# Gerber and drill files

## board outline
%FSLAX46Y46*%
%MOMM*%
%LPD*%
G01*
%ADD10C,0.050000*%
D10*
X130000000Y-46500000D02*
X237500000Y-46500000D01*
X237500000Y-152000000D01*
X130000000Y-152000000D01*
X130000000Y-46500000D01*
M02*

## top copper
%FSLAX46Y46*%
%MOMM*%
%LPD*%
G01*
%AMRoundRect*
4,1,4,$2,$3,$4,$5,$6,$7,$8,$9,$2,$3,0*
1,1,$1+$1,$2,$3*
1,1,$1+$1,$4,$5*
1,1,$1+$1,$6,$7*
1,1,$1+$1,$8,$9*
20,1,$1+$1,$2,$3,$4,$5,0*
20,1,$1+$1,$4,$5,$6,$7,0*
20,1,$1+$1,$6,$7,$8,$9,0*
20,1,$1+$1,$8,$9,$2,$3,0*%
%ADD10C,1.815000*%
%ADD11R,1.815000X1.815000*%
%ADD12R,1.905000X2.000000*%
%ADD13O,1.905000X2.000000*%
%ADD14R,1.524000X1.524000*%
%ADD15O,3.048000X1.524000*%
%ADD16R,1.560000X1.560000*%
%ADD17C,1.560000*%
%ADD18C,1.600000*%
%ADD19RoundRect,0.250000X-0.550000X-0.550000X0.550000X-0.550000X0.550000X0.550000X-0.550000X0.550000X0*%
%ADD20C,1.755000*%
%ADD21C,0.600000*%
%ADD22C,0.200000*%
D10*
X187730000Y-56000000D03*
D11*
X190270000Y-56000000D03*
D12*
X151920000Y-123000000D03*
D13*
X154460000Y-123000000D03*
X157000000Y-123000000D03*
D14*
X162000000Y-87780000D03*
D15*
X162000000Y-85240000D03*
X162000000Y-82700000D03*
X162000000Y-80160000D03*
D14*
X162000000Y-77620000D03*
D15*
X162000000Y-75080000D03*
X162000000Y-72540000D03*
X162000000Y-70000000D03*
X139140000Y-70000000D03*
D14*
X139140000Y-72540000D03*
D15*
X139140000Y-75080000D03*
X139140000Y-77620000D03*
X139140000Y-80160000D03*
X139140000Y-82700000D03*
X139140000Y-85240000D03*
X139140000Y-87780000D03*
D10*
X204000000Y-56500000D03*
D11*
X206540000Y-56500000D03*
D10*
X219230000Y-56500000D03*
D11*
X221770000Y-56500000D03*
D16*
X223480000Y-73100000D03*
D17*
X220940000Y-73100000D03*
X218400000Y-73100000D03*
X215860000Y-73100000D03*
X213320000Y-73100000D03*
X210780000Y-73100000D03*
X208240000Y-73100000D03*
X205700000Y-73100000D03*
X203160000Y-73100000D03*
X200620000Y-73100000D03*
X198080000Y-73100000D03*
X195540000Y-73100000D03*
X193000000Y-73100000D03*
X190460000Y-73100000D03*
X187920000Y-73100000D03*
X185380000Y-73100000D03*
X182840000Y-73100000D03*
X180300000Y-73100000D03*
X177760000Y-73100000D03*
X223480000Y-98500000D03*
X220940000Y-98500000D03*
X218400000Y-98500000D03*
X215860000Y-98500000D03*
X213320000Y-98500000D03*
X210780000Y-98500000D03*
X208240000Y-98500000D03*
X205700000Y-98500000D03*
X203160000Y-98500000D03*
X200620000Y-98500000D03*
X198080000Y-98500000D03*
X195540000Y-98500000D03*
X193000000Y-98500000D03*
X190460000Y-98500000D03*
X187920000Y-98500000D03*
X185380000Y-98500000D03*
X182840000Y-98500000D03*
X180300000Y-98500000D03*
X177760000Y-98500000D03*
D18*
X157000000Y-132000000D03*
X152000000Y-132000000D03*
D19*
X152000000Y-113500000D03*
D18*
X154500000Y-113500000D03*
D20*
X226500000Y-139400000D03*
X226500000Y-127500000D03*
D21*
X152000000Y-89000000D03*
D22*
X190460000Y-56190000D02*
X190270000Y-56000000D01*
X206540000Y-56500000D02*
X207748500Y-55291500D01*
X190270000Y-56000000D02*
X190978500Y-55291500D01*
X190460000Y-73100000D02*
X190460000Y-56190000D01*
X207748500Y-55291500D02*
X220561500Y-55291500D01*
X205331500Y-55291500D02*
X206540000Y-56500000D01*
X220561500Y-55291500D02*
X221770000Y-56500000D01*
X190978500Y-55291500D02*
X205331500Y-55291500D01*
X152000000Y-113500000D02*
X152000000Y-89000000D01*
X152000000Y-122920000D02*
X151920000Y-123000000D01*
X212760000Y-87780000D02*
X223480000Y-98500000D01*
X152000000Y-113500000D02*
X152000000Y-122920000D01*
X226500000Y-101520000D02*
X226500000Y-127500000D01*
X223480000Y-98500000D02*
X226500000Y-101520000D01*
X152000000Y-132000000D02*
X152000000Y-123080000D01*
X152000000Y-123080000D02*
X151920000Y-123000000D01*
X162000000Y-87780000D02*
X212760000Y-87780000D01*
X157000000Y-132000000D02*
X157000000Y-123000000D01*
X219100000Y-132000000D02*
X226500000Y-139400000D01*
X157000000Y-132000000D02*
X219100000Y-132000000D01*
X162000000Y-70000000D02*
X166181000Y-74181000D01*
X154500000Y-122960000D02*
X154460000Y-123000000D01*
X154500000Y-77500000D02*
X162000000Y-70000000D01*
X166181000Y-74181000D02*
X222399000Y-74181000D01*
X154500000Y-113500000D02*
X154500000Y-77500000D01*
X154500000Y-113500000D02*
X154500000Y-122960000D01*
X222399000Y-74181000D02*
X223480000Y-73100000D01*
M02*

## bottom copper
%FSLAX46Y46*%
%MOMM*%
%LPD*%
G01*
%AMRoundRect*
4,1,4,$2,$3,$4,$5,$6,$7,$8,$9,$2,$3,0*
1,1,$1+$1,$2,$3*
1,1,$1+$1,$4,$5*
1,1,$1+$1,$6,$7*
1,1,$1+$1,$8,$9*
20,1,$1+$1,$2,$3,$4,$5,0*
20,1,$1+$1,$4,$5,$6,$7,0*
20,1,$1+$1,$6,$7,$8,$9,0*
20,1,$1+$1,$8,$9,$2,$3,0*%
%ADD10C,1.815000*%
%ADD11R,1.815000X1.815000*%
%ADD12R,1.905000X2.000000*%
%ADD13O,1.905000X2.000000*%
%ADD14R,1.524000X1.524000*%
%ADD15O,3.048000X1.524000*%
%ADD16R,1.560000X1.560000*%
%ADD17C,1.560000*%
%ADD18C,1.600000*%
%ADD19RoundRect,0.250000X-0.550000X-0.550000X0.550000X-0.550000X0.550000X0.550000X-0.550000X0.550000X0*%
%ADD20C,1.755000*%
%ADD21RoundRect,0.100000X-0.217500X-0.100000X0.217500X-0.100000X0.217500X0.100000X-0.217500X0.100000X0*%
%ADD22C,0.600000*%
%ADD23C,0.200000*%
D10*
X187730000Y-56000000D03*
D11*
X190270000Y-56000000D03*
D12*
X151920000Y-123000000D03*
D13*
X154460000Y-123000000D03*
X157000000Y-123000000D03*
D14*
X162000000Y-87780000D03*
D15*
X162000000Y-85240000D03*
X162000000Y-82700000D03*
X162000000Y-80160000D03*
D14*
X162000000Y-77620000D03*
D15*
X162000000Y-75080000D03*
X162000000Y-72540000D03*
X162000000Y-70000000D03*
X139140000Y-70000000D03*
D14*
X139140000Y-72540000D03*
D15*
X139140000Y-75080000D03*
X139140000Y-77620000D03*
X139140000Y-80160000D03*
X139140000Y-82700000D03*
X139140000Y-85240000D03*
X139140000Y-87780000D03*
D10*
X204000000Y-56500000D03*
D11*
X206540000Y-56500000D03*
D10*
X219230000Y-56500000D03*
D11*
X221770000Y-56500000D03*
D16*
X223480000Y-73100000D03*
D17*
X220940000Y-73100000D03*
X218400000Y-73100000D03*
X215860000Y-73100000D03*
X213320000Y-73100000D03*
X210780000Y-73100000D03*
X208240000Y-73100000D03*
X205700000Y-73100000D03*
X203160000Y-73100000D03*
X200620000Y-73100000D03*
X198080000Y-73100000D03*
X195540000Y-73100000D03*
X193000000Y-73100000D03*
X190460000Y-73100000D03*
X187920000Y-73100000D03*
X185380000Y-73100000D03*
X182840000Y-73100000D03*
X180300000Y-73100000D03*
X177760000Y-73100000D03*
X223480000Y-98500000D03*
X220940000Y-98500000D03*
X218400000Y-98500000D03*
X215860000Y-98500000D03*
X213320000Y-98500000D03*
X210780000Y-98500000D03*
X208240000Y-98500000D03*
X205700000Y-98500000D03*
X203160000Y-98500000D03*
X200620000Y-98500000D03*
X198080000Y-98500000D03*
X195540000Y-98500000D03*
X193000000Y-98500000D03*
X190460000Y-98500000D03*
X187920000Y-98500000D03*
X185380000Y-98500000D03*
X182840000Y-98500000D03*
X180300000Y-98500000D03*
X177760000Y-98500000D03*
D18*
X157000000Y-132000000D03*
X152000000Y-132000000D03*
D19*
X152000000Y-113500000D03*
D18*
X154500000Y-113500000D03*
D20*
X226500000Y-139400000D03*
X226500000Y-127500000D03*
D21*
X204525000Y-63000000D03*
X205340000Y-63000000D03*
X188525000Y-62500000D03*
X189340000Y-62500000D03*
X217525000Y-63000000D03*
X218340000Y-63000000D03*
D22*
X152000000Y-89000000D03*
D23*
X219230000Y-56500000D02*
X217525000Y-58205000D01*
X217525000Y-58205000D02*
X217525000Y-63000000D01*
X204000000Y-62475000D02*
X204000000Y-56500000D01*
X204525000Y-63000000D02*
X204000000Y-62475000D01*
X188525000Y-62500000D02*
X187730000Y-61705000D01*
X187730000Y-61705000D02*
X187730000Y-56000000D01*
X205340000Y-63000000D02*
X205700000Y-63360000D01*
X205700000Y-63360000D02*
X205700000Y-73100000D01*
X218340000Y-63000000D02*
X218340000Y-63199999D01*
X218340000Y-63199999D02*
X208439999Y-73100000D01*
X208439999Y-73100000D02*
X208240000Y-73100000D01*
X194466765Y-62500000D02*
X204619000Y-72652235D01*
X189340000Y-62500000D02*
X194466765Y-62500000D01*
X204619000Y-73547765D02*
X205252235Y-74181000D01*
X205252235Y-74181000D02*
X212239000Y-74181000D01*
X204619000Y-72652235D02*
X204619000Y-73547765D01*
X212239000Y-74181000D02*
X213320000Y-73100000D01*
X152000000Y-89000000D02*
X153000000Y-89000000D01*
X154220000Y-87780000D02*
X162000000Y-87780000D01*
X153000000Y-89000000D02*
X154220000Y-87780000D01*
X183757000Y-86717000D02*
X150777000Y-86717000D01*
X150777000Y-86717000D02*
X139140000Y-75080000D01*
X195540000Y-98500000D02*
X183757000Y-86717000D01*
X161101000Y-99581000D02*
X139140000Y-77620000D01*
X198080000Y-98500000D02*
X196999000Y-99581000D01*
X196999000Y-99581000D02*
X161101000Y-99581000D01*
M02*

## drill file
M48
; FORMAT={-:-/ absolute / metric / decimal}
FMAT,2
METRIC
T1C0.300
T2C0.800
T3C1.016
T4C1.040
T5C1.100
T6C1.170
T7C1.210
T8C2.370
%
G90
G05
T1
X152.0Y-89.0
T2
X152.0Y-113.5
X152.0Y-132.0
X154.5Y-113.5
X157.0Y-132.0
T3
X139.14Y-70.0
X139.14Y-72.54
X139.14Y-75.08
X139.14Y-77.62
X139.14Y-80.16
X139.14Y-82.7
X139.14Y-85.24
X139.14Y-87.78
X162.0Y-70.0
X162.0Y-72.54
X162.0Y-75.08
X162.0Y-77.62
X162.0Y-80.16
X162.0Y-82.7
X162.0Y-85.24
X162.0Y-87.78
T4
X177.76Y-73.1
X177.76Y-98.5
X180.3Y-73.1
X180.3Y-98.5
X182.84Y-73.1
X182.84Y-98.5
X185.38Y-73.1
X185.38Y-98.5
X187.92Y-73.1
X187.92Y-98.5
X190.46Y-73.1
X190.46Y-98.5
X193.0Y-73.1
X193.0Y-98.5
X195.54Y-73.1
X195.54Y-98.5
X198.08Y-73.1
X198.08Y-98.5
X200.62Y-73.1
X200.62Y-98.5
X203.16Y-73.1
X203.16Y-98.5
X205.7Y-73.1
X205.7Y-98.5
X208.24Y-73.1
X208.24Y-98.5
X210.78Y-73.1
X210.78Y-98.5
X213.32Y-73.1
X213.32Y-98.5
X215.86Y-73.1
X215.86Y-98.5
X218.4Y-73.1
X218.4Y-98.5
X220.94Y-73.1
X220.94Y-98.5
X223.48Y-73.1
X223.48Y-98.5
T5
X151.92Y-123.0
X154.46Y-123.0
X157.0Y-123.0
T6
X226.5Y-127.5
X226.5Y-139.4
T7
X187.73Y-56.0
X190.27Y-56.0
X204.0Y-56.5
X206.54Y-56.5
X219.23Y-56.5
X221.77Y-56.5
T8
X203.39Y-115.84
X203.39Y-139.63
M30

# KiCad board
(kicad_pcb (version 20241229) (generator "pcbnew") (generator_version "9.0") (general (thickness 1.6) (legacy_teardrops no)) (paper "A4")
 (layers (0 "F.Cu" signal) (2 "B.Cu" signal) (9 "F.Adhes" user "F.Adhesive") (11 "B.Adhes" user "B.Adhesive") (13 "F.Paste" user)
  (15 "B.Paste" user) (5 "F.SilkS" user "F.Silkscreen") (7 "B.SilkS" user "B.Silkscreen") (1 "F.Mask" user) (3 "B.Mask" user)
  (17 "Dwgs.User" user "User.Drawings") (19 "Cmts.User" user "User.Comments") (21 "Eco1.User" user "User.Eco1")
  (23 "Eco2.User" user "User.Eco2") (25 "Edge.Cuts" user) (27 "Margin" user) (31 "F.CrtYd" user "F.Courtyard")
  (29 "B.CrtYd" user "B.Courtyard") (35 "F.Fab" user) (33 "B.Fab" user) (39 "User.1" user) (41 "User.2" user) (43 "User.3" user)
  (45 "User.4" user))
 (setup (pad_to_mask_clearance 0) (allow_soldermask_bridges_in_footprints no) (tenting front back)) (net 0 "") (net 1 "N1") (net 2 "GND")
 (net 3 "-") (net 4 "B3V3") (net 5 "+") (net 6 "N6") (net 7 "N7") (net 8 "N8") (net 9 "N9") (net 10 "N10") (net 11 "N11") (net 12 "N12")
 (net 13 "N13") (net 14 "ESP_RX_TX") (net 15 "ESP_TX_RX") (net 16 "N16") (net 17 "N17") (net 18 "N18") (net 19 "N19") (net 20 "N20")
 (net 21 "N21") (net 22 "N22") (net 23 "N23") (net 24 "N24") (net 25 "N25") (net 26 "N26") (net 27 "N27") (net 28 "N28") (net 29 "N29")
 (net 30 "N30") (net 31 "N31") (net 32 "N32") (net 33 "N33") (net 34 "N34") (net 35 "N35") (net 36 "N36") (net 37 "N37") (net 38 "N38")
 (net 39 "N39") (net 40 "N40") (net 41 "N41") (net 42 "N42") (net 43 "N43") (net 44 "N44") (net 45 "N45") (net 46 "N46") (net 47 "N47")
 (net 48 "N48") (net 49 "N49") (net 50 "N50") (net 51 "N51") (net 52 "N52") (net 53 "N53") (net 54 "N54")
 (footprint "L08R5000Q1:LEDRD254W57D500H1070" (layer "F.Cu") (at 189 56 180)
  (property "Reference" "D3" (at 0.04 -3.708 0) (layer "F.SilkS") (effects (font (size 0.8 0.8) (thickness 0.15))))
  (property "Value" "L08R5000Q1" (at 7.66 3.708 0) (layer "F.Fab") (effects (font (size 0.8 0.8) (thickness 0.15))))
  (pad "A" thru_hole circle (at 1.27 0 180) (size 1.815 1.815) (drill 1.21) (layers "*.Cu" "*.Mask") (remove_unused_layers no) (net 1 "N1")
   (solder_mask_margin 0.102))
  (pad "C" thru_hole rect (at -1.27 0 180) (size 1.815 1.815) (drill 1.21) (layers "*.Cu" "*.Mask") (remove_unused_layers no) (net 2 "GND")
   (solder_mask_margin 0.102)))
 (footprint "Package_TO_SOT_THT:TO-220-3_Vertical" (layer "F.Cu") (at 151.92 123)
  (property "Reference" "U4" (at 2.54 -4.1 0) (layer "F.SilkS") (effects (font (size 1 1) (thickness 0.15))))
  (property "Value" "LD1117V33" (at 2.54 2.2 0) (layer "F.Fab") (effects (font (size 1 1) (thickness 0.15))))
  (pad "1" thru_hole rect (at 0 0) (size 1.905 2) (drill 1.1) (layers "*.Cu" "*.Mask") (remove_unused_layers no) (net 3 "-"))
  (pad "2" thru_hole oval (at 2.54 0) (size 1.905 2) (drill 1.1) (layers "*.Cu" "*.Mask") (remove_unused_layers no) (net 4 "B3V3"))
  (pad "3" thru_hole oval (at 5.08 0) (size 1.905 2) (drill 1.1) (layers "*.Cu" "*.Mask") (remove_unused_layers no) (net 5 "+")))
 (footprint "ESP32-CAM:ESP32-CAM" (layer "F.Cu") (at 150.57 80.16 180)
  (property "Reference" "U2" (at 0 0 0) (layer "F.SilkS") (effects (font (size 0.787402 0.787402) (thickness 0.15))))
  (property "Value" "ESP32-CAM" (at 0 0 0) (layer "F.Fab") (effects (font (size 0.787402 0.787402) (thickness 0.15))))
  (pad "P$1" thru_hole rect (at -11.43 -7.62 180) (size 1.524 1.524) (drill 1.016) (layers "*.Cu" "*.Mask") (remove_unused_layers no)
   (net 3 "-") (solder_mask_margin 0.102))
  (pad "P$2" thru_hole oval (at -11.43 -5.08 180) (size 3.048 1.524) (drill 1.016) (layers "*.Cu" "*.Mask") (remove_unused_layers no)
   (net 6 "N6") (solder_mask_margin 0.102))
  (pad "P$3" thru_hole oval (at -11.43 -2.54 180) (size 3.048 1.524) (drill 1.016) (layers "*.Cu" "*.Mask") (remove_unused_layers no)
   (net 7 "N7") (solder_mask_margin 0.102))
  (pad "P$4" thru_hole oval (at -11.43 0 180) (size 3.048 1.524) (drill 1.016) (layers "*.Cu" "*.Mask") (remove_unused_layers no)
   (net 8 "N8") (solder_mask_margin 0.102))
  (pad "P$5" thru_hole rect (at -11.43 2.54 180) (size 1.524 1.524) (drill 1.016) (layers "*.Cu" "*.Mask") (remove_unused_layers no)
   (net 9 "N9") (solder_mask_margin 0.102))
  (pad "P$6" thru_hole oval (at -11.43 5.08 180) (size 3.048 1.524) (drill 1.016) (layers "*.Cu" "*.Mask") (remove_unused_layers no)
   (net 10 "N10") (solder_mask_margin 0.102))
  (pad "P$7" thru_hole oval (at -11.43 7.62 180) (size 3.048 1.524) (drill 1.016) (layers "*.Cu" "*.Mask") (remove_unused_layers no)
   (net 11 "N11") (solder_mask_margin 0.102))
  (pad "P$8" thru_hole oval (at -11.43 10.16 180) (size 3.048 1.524) (drill 1.016) (layers "*.Cu" "*.Mask") (remove_unused_layers no)
   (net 4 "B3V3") (solder_mask_margin 0.102))
  (pad "P$9" thru_hole oval (at 11.43 10.16 180) (size 3.048 1.524) (drill 1.016) (layers "*.Cu" "*.Mask") (remove_unused_layers no)
   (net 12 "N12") (solder_mask_margin 0.102))
  (pad "P$10" thru_hole rect (at 11.43 7.62 180) (size 1.524 1.524) (drill 1.016) (layers "*.Cu" "*.Mask") (remove_unused_layers no)
   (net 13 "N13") (solder_mask_margin 0.102))
  (pad "P$11" thru_hole oval (at 11.43 5.08 180) (size 3.048 1.524) (drill 1.016) (layers "*.Cu" "*.Mask") (remove_unused_layers no)
   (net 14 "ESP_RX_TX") (solder_mask_margin 0.102))
  (pad "P$12" thru_hole oval (at 11.43 2.54 180) (size 3.048 1.524) (drill 1.016) (layers "*.Cu" "*.Mask") (remove_unused_layers no)
   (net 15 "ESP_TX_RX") (solder_mask_margin 0.102))
  (pad "P$13" thru_hole oval (at 11.43 0 180) (size 3.048 1.524) (drill 1.016) (layers "*.Cu" "*.Mask") (remove_unused_layers no)
   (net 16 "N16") (solder_mask_margin 0.102))
  (pad "P$14" thru_hole oval (at 11.43 -2.54 180) (size 3.048 1.524) (drill 1.016) (layers "*.Cu" "*.Mask") (remove_unused_layers no)
   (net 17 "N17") (solder_mask_margin 0.102))
  (pad "P$15" thru_hole oval (at 11.43 -5.08 180) (size 3.048 1.524) (drill 1.016) (layers "*.Cu" "*.Mask") (remove_unused_layers no)
   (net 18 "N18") (solder_mask_margin 0.102))
  (pad "P$16" thru_hole oval (at 11.43 -7.62 180) (size 3.048 1.524) (drill 1.016) (layers "*.Cu" "*.Mask") (remove_unused_layers no)
   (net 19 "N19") (solder_mask_margin 0.102)))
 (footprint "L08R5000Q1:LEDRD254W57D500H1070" (layer "F.Cu") (at 205.27 56.5 180)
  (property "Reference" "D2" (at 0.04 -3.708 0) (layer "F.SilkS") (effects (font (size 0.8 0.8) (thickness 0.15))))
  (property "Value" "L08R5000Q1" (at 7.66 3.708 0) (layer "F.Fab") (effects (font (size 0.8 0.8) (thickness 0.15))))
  (pad "A" thru_hole circle (at 1.27 0 180) (size 1.815 1.815) (drill 1.21) (layers "*.Cu" "*.Mask") (remove_unused_layers no)
   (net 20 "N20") (solder_mask_margin 0.102))
  (pad "C" thru_hole rect (at -1.27 0 180) (size 1.815 1.815) (drill 1.21) (layers "*.Cu" "*.Mask") (remove_unused_layers no) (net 2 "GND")
   (solder_mask_margin 0.102)))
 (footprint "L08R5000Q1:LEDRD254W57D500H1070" (layer "F.Cu") (at 220.5 56.5 180)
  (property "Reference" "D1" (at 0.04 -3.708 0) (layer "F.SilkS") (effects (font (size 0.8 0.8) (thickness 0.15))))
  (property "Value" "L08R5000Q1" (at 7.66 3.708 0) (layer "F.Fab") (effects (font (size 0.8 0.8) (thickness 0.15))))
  (pad "A" thru_hole circle (at 1.27 0 180) (size 1.815 1.815) (drill 1.21) (layers "*.Cu" "*.Mask") (remove_unused_layers no)
   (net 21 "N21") (solder_mask_margin 0.102))
  (pad "C" thru_hole rect (at -1.27 0 180) (size 1.815 1.815) (drill 1.21) (layers "*.Cu" "*.Mask") (remove_unused_layers no) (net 2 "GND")
   (solder_mask_margin 0.102)))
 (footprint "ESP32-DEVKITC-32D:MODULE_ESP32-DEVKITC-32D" (layer "F.Cu") (at 203.72 85.8 -90)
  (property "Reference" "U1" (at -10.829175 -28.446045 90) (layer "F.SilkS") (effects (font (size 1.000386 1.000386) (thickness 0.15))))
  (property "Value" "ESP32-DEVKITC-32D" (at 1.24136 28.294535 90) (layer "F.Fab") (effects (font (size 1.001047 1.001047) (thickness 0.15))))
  (pad "J2-1" thru_hole rect (at -12.7 -19.76 270) (size 1.56 1.56) (drill 1.04) (layers "*.Cu" "*.Mask") (remove_unused_layers no)
   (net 4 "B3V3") (solder_mask_margin 0.102))
  (pad "J2-2" thru_hole circle (at -12.7 -17.22 270) (size 1.56 1.56) (drill 1.04) (layers "*.Cu" "*.Mask") (remove_unused_layers no)
   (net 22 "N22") (solder_mask_margin 0.102))
  (pad "J2-3" thru_hole circle (at -12.7 -14.68 270) (size 1.56 1.56) (drill 1.04) (layers "*.Cu" "*.Mask") (remove_unused_layers no)
   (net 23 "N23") (solder_mask_margin 0.102))
  (pad "J2-4" thru_hole circle (at -12.7 -12.14 270) (size 1.56 1.56) (drill 1.04) (layers "*.Cu" "*.Mask") (remove_unused_layers no)
   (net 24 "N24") (solder_mask_margin 0.102))
  (pad "J2-5" thru_hole circle (at -12.7 -9.6 270) (size 1.56 1.56) (drill 1.04) (layers "*.Cu" "*.Mask") (remove_unused_layers no)
   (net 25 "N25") (solder_mask_margin 0.102))
  (pad "J2-6" thru_hole circle (at -12.7 -7.06 270) (size 1.56 1.56) (drill 1.04) (layers "*.Cu" "*.Mask") (remove_unused_layers no)
   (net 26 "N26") (solder_mask_margin 0.102))
  (pad "J2-7" thru_hole circle (at -12.7 -4.52 270) (size 1.56 1.56) (drill 1.04) (layers "*.Cu" "*.Mask") (remove_unused_layers no)
   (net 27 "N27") (solder_mask_margin 0.102))
  (pad "J2-8" thru_hole circle (at -12.7 -1.98 270) (size 1.56 1.56) (drill 1.04) (layers "*.Cu" "*.Mask") (remove_unused_layers no)
   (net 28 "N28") (solder_mask_margin 0.102))
  (pad "J2-9" thru_hole circle (at -12.7 0.56 270) (size 1.56 1.56) (drill 1.04) (layers "*.Cu" "*.Mask") (remove_unused_layers no)
   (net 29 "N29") (solder_mask_margin 0.102))
  (pad "J2-10" thru_hole circle (at -12.7 3.1 270) (size 1.56 1.56) (drill 1.04) (layers "*.Cu" "*.Mask") (remove_unused_layers no)
   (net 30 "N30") (solder_mask_margin 0.102))
  (pad "J2-11" thru_hole circle (at -12.7 5.64 270) (size 1.56 1.56) (drill 1.04) (layers "*.Cu" "*.Mask") (remove_unused_layers no)
   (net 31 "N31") (solder_mask_margin 0.102))
  (pad "J2-12" thru_hole circle (at -12.7 8.18 270) (size 1.56 1.56) (drill 1.04) (layers "*.Cu" "*.Mask") (remove_unused_layers no)
   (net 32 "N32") (solder_mask_margin 0.102))
  (pad "J2-13" thru_hole circle (at -12.7 10.72 270) (size 1.56 1.56) (drill 1.04) (layers "*.Cu" "*.Mask") (remove_unused_layers no)
   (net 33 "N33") (solder_mask_margin 0.102))
  (pad "J2-14" thru_hole circle (at -12.7 13.26 270) (size 1.56 1.56) (drill 1.04) (layers "*.Cu" "*.Mask") (remove_unused_layers no)
   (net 2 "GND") (solder_mask_margin 0.102))
  (pad "J2-15" thru_hole circle (at -12.7 15.8 270) (size 1.56 1.56) (drill 1.04) (layers "*.Cu" "*.Mask") (remove_unused_layers no)
   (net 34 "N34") (solder_mask_margin 0.102))
  (pad "J2-16" thru_hole circle (at -12.7 18.34 270) (size 1.56 1.56) (drill 1.04) (layers "*.Cu" "*.Mask") (remove_unused_layers no)
   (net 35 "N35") (solder_mask_margin 0.102))
  (pad "J2-17" thru_hole circle (at -12.7 20.88 270) (size 1.56 1.56) (drill 1.04) (layers "*.Cu" "*.Mask") (remove_unused_layers no)
   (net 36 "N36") (solder_mask_margin 0.102))
  (pad "J2-18" thru_hole circle (at -12.7 23.42 270) (size 1.56 1.56) (drill 1.04) (layers "*.Cu" "*.Mask") (remove_unused_layers no)
   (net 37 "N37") (solder_mask_margin 0.102))
  (pad "J2-19" thru_hole circle (at -12.7 25.96 270) (size 1.56 1.56) (drill 1.04) (layers "*.Cu" "*.Mask") (remove_unused_layers no)
   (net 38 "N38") (solder_mask_margin 0.102))
  (pad "J3-1" thru_hole circle (at 12.7 -19.76 270) (size 1.56 1.56) (drill 1.04) (layers "*.Cu" "*.Mask") (remove_unused_layers no)
   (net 3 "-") (solder_mask_margin 0.102))
  (pad "J3-2" thru_hole circle (at 12.7 -17.22 270) (size 1.56 1.56) (drill 1.04) (layers "*.Cu" "*.Mask") (remove_unused_layers no)
   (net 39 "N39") (solder_mask_margin 0.102))
  (pad "J3-3" thru_hole circle (at 12.7 -14.68 270) (size 1.56 1.56) (drill 1.04) (layers "*.Cu" "*.Mask") (remove_unused_layers no)
   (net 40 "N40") (solder_mask_margin 0.102))
  (pad "J3-4" thru_hole circle (at 12.7 -12.14 270) (size 1.56 1.56) (drill 1.04) (layers "*.Cu" "*.Mask") (remove_unused_layers no)
   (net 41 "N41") (solder_mask_margin 0.102))
  (pad "J3-5" thru_hole circle (at 12.7 -9.6 270) (size 1.56 1.56) (drill 1.04) (layers "*.Cu" "*.Mask") (remove_unused_layers no)
   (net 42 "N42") (solder_mask_margin 0.102))
  (pad "J3-6" thru_hole circle (at 12.7 -7.06 270) (size 1.56 1.56) (drill 1.04) (layers "*.Cu" "*.Mask") (remove_unused_layers no)
   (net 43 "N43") (solder_mask_margin 0.102))
  (pad "J3-7" thru_hole circle (at 12.7 -4.52 270) (size 1.56 1.56) (drill 1.04) (layers "*.Cu" "*.Mask") (remove_unused_layers no)
   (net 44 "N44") (solder_mask_margin 0.102))
  (pad "J3-8" thru_hole circle (at 12.7 -1.98 270) (size 1.56 1.56) (drill 1.04) (layers "*.Cu" "*.Mask") (remove_unused_layers no)
   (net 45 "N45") (solder_mask_margin 0.102))
  (pad "J3-9" thru_hole circle (at 12.7 0.56 270) (size 1.56 1.56) (drill 1.04) (layers "*.Cu" "*.Mask") (remove_unused_layers no)
   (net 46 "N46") (solder_mask_margin 0.102))
  (pad "J3-10" thru_hole circle (at 12.7 3.1 270) (size 1.56 1.56) (drill 1.04) (layers "*.Cu" "*.Mask") (remove_unused_layers no)
   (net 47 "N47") (solder_mask_margin 0.102))
  (pad "J3-11" thru_hole circle (at 12.7 5.64 270) (size 1.56 1.56) (drill 1.04) (layers "*.Cu" "*.Mask") (remove_unused_layers no)
   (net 15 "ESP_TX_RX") (solder_mask_margin 0.102))
  (pad "J3-12" thru_hole circle (at 12.7 8.18 270) (size 1.56 1.56) (drill 1.04) (layers "*.Cu" "*.Mask") (remove_unused_layers no)
   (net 14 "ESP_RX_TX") (solder_mask_margin 0.102))
  (pad "J3-13" thru_hole circle (at 12.7 10.72 270) (size 1.56 1.56) (drill 1.04) (layers "*.Cu" "*.Mask") (remove_unused_layers no)
   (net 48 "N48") (solder_mask_margin 0.102))
  (pad "J3-14" thru_hole circle (at 12.7 13.26 270) (size 1.56 1.56) (drill 1.04) (layers "*.Cu" "*.Mask") (remove_unused_layers no)
   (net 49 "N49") (solder_mask_margin 0.102))
  (pad "J3-15" thru_hole circle (at 12.7 15.8 270) (size 1.56 1.56) (drill 1.04) (layers "*.Cu" "*.Mask") (remove_unused_layers no)
   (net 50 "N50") (solder_mask_margin 0.102))
  (pad "J3-16" thru_hole circle (at 12.7 18.34 270) (size 1.56 1.56) (drill 1.04) (layers "*.Cu" "*.Mask") (remove_unused_layers no)
   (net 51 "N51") (solder_mask_margin 0.102))
  (pad "J3-17" thru_hole circle (at 12.7 20.88 270) (size 1.56 1.56) (drill 1.04) (layers "*.Cu" "*.Mask") (remove_unused_layers no)
   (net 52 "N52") (solder_mask_margin 0.102))
  (pad "J3-18" thru_hole circle (at 12.7 23.42 270) (size 1.56 1.56) (drill 1.04) (layers "*.Cu" "*.Mask") (remove_unused_layers no)
   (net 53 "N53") (solder_mask_margin 0.102))
  (pad "J3-19" thru_hole circle (at 12.7 25.96 270) (size 1.56 1.56) (drill 1.04) (layers "*.Cu" "*.Mask") (remove_unused_layers no)
   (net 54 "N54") (solder_mask_margin 0.102)))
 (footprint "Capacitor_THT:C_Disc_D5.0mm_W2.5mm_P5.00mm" (layer "F.Cu") (at 157 132 180)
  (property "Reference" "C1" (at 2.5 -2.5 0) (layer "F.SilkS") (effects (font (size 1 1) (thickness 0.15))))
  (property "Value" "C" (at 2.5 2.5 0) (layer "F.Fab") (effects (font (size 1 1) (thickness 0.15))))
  (pad "1" thru_hole circle (at 0 0 180) (size 1.6 1.6) (drill 0.8) (layers "*.Cu" "*.Mask") (remove_unused_layers no) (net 5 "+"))
  (pad "2" thru_hole circle (at 5 0 180) (size 1.6 1.6) (drill 0.8) (layers "*.Cu" "*.Mask") (remove_unused_layers no) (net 3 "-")))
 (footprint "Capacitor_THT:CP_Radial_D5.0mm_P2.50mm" (layer "F.Cu") (at 152 113.5)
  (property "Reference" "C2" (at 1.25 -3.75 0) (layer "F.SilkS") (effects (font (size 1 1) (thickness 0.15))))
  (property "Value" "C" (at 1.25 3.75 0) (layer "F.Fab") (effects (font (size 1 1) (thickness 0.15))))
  (pad "1" thru_hole roundrect (at 0 0) (size 1.6 1.6) (drill 0.8) (layers "*.Cu" "*.Mask") (remove_unused_layers no)
   (roundrect_rratio 0.15625) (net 3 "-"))
  (pad "2" thru_hole circle (at 2.5 0) (size 1.6 1.6) (drill 0.8) (layers "*.Cu" "*.Mask") (remove_unused_layers no) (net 4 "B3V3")))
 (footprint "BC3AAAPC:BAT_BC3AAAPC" (layer "F.Cu") (at 203.39 127.23)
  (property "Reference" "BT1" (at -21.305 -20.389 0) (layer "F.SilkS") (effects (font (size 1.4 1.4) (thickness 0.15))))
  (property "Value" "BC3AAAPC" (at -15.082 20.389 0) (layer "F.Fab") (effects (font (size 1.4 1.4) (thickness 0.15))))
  (pad "" np_thru_hole circle (at 0 -11.39) (size 2.37 2.37) (drill 2.37) (layers "*.Cu" "*.Mask"))
  (pad "" np_thru_hole circle (at 0 12.4) (size 2.37 2.37) (drill 2.37) (layers "*.Cu" "*.Mask"))
  (pad "+" thru_hole circle (at 23.11 12.17) (size 1.755 1.755) (drill 1.17) (layers "*.Cu" "*.Mask") (remove_unused_layers no) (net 5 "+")
   (solder_mask_margin 0.102))
  (pad "-" thru_hole circle (at 23.11 0.27) (size 1.755 1.755) (drill 1.17) (layers "*.Cu" "*.Mask") (remove_unused_layers no) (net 3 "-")
   (solder_mask_margin 0.102)))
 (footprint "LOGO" (layer "F.Cu") (at 137 52.5)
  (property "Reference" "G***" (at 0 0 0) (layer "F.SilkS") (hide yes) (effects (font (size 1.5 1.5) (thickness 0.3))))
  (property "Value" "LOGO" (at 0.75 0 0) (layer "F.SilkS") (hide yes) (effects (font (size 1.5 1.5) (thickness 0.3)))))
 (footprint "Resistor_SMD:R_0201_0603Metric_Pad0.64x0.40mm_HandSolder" (layer "B.Cu") (at 204.9325 63)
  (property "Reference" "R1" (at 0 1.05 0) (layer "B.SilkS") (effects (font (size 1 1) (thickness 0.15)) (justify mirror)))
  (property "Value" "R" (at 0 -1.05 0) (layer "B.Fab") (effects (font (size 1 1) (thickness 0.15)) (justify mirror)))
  (pad "" smd roundrect (at -0.4325 0) (size 0.458 0.36) (layers "B.Paste") (roundrect_rratio 0.25))
  (pad "" smd roundrect (at 0.4325 0) (size 0.458 0.36) (layers "B.Paste") (roundrect_rratio 0.25))
  (pad "1" smd roundrect (at -0.4075 0) (size 0.635 0.4) (layers "B.Cu" "B.Mask") (roundrect_rratio 0.25) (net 20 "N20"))
  (pad "2" smd roundrect (at 0.4075 0) (size 0.635 0.4) (layers "B.Cu" "B.Mask") (roundrect_rratio 0.25) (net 28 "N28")))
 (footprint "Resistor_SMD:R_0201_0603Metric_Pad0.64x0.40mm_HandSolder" (layer "B.Cu") (at 188.9325 62.5)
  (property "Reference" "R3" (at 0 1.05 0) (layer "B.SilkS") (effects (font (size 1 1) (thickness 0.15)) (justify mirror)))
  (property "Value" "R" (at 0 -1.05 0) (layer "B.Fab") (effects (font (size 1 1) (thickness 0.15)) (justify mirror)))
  (pad "" smd roundrect (at -0.4325 0) (size 0.458 0.36) (layers "B.Paste") (roundrect_rratio 0.25))
  (pad "" smd roundrect (at 0.4325 0) (size 0.458 0.36) (layers "B.Paste") (roundrect_rratio 0.25))
  (pad "1" smd roundrect (at -0.4075 0) (size 0.635 0.4) (layers "B.Cu" "B.Mask") (roundrect_rratio 0.25) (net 1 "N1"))
  (pad "2" smd roundrect (at 0.4075 0) (size 0.635 0.4) (layers "B.Cu" "B.Mask") (roundrect_rratio 0.25) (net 25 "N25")))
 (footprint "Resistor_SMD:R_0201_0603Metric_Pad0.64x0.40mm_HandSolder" (layer "B.Cu") (at 217.9325 63)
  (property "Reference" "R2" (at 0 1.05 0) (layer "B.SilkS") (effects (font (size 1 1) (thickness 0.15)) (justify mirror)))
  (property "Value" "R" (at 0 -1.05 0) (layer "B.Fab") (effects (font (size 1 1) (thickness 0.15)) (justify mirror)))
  (pad "" smd roundrect (at -0.4325 0) (size 0.458 0.36) (layers "B.Paste") (roundrect_rratio 0.25))
  (pad "" smd roundrect (at 0.4325 0) (size 0.458 0.36) (layers "B.Paste") (roundrect_rratio 0.25))
  (pad "1" smd roundrect (at -0.4075 0) (size 0.635 0.4) (layers "B.Cu" "B.Mask") (roundrect_rratio 0.25) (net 21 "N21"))
  (pad "2" smd roundrect (at 0.4075 0) (size 0.635 0.4) (layers "B.Cu" "B.Mask") (roundrect_rratio 0.25) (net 27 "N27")))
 (gr_rect (start 130 46.5) (end 237.5 152) (stroke (width 0.05) (type default)) (fill no) (layer "Edge.Cuts"))
 (segment (start 219.23 56.5) (end 217.525 58.205) (width 0.2) (layer "B.Cu") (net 21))
 (segment (start 217.525 58.205) (end 217.525 63) (width 0.2) (layer "B.Cu") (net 21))
 (segment (start 190.46 56.19) (end 190.27 56) (width 0.2) (layer "F.Cu") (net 2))
 (segment (start 206.54 56.5) (end 207.7485 55.2915) (width 0.2) (layer "F.Cu") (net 2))
 (segment (start 190.27 56) (end 190.9785 55.2915) (width 0.2) (layer "F.Cu") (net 2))
 (segment (start 190.46 73.1) (end 190.46 56.19) (width 0.2) (layer "F.Cu") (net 2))
 (segment (start 207.7485 55.2915) (end 220.5615 55.2915) (width 0.2) (layer "F.Cu") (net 2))
 (segment (start 205.3315 55.2915) (end 206.54 56.5) (width 0.2) (layer "F.Cu") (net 2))
 (segment (start 220.5615 55.2915) (end 221.77 56.5) (width 0.2) (layer "F.Cu") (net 2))
 (segment (start 190.9785 55.2915) (end 205.3315 55.2915) (width 0.2) (layer "F.Cu") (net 2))
 (segment (start 204 62.475) (end 204 56.5) (width 0.2) (layer "B.Cu") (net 20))
 (segment (start 204.525 63) (end 204 62.475) (width 0.2) (layer "B.Cu") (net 20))
 (segment (start 188.525 62.5) (end 187.73 61.705) (width 0.2) (layer "B.Cu") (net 1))
 (segment (start 187.73 61.705) (end 187.73 56) (width 0.2) (layer "B.Cu") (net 1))
 (segment (start 205.34 63) (end 205.7 63.36) (width 0.2) (layer "B.Cu") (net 28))
 (segment (start 205.7 63.36) (end 205.7 73.1) (width 0.2) (layer "B.Cu") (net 28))
 (segment (start 218.34 63) (end 218.34 63.199999) (width 0.2) (layer "B.Cu") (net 27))
 (segment (start 218.34 63.199999) (end 208.439999 73.1) (width 0.2) (layer "B.Cu") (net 27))
 (segment (start 208.439999 73.1) (end 208.24 73.1) (width 0.2) (layer "B.Cu") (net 27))
 (segment (start 194.466765 62.5) (end 204.619 72.652235) (width 0.2) (layer "B.Cu") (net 25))
 (segment (start 189.34 62.5) (end 194.466765 62.5) (width 0.2) (layer "B.Cu") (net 25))
 (segment (start 204.619 73.547765) (end 205.252235 74.181) (width 0.2) (layer "B.Cu") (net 25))
 (segment (start 205.252235 74.181) (end 212.239 74.181) (width 0.2) (layer "B.Cu") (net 25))
 (segment (start 204.619 72.652235) (end 204.619 73.547765) (width 0.2) (layer "B.Cu") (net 25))
 (segment (start 212.239 74.181) (end 213.32 73.1) (width 0.2) (layer "B.Cu") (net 25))
 (segment (start 152 113.5) (end 152 89) (width 0.2) (layer "F.Cu") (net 3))
 (segment (start 152 122.92) (end 151.92 123) (width 0.2) (layer "F.Cu") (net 3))
 (segment (start 212.76 87.78) (end 223.48 98.5) (width 0.2) (layer "F.Cu") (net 3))
 (segment (start 152 113.5) (end 152 122.92) (width 0.2) (layer "F.Cu") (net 3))
 (segment (start 226.5 101.52) (end 226.5 127.5) (width 0.2) (layer "F.Cu") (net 3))
 (segment (start 223.48 98.5) (end 226.5 101.52) (width 0.2) (layer "F.Cu") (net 3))
 (segment (start 152 132) (end 152 123.08) (width 0.2) (layer "F.Cu") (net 3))
 (segment (start 152 123.08) (end 151.92 123) (width 0.2) (layer "F.Cu") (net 3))
 (segment (start 162 87.78) (end 212.76 87.78) (width 0.2) (layer "F.Cu") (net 3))
 (via (at 152 89) (size 0.6) (drill 0.3) (layers "F.Cu" "B.Cu") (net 3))
 (segment (start 152 89) (end 153 89) (width 0.2) (layer "B.Cu") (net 3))
 (segment (start 154.22 87.78) (end 162 87.78) (width 0.2) (layer "B.Cu") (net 3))
 (segment (start 153 89) (end 154.22 87.78) (width 0.2) (layer "B.Cu") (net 3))
 (segment (start 157 132) (end 157 123) (width 0.2) (layer "F.Cu") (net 5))
 (segment (start 219.1 132) (end 226.5 139.4) (width 0.2) (layer "F.Cu") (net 5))
 (segment (start 157 132) (end 219.1 132) (width 0.2) (layer "F.Cu") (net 5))
 (segment (start 162 70) (end 166.181 74.181) (width 0.2) (layer "F.Cu") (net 4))
 (segment (start 154.5 122.96) (end 154.46 123) (width 0.2) (layer "F.Cu") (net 4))
 (segment (start 154.5 77.5) (end 162 70) (width 0.2) (layer "F.Cu") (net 4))
 (segment (start 166.181 74.181) (end 222.399 74.181) (width 0.2) (layer "F.Cu") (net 4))
 (segment (start 154.5 113.5) (end 154.5 77.5) (width 0.2) (layer "F.Cu") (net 4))
 (segment (start 154.5 113.5) (end 154.5 122.96) (width 0.2) (layer "F.Cu") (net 4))
 (segment (start 222.399 74.181) (end 223.48 73.1) (width 0.2) (layer "F.Cu") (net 4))
 (segment (start 183.757 86.717) (end 150.777 86.717) (width 0.2) (layer "B.Cu") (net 14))
 (segment (start 150.777 86.717) (end 139.14 75.08) (width 0.2) (layer "B.Cu") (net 14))
 (segment (start 195.54 98.5) (end 183.757 86.717) (width 0.2) (layer "B.Cu") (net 14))
 (segment (start 161.101 99.581) (end 139.14 77.62) (width 0.2) (layer "B.Cu") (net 15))
 (segment (start 198.08 98.5) (end 196.999 99.581) (width 0.2) (layer "B.Cu") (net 15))
 (segment (start 196.999 99.581) (end 161.101 99.581) (width 0.2) (layer "B.Cu") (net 15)))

